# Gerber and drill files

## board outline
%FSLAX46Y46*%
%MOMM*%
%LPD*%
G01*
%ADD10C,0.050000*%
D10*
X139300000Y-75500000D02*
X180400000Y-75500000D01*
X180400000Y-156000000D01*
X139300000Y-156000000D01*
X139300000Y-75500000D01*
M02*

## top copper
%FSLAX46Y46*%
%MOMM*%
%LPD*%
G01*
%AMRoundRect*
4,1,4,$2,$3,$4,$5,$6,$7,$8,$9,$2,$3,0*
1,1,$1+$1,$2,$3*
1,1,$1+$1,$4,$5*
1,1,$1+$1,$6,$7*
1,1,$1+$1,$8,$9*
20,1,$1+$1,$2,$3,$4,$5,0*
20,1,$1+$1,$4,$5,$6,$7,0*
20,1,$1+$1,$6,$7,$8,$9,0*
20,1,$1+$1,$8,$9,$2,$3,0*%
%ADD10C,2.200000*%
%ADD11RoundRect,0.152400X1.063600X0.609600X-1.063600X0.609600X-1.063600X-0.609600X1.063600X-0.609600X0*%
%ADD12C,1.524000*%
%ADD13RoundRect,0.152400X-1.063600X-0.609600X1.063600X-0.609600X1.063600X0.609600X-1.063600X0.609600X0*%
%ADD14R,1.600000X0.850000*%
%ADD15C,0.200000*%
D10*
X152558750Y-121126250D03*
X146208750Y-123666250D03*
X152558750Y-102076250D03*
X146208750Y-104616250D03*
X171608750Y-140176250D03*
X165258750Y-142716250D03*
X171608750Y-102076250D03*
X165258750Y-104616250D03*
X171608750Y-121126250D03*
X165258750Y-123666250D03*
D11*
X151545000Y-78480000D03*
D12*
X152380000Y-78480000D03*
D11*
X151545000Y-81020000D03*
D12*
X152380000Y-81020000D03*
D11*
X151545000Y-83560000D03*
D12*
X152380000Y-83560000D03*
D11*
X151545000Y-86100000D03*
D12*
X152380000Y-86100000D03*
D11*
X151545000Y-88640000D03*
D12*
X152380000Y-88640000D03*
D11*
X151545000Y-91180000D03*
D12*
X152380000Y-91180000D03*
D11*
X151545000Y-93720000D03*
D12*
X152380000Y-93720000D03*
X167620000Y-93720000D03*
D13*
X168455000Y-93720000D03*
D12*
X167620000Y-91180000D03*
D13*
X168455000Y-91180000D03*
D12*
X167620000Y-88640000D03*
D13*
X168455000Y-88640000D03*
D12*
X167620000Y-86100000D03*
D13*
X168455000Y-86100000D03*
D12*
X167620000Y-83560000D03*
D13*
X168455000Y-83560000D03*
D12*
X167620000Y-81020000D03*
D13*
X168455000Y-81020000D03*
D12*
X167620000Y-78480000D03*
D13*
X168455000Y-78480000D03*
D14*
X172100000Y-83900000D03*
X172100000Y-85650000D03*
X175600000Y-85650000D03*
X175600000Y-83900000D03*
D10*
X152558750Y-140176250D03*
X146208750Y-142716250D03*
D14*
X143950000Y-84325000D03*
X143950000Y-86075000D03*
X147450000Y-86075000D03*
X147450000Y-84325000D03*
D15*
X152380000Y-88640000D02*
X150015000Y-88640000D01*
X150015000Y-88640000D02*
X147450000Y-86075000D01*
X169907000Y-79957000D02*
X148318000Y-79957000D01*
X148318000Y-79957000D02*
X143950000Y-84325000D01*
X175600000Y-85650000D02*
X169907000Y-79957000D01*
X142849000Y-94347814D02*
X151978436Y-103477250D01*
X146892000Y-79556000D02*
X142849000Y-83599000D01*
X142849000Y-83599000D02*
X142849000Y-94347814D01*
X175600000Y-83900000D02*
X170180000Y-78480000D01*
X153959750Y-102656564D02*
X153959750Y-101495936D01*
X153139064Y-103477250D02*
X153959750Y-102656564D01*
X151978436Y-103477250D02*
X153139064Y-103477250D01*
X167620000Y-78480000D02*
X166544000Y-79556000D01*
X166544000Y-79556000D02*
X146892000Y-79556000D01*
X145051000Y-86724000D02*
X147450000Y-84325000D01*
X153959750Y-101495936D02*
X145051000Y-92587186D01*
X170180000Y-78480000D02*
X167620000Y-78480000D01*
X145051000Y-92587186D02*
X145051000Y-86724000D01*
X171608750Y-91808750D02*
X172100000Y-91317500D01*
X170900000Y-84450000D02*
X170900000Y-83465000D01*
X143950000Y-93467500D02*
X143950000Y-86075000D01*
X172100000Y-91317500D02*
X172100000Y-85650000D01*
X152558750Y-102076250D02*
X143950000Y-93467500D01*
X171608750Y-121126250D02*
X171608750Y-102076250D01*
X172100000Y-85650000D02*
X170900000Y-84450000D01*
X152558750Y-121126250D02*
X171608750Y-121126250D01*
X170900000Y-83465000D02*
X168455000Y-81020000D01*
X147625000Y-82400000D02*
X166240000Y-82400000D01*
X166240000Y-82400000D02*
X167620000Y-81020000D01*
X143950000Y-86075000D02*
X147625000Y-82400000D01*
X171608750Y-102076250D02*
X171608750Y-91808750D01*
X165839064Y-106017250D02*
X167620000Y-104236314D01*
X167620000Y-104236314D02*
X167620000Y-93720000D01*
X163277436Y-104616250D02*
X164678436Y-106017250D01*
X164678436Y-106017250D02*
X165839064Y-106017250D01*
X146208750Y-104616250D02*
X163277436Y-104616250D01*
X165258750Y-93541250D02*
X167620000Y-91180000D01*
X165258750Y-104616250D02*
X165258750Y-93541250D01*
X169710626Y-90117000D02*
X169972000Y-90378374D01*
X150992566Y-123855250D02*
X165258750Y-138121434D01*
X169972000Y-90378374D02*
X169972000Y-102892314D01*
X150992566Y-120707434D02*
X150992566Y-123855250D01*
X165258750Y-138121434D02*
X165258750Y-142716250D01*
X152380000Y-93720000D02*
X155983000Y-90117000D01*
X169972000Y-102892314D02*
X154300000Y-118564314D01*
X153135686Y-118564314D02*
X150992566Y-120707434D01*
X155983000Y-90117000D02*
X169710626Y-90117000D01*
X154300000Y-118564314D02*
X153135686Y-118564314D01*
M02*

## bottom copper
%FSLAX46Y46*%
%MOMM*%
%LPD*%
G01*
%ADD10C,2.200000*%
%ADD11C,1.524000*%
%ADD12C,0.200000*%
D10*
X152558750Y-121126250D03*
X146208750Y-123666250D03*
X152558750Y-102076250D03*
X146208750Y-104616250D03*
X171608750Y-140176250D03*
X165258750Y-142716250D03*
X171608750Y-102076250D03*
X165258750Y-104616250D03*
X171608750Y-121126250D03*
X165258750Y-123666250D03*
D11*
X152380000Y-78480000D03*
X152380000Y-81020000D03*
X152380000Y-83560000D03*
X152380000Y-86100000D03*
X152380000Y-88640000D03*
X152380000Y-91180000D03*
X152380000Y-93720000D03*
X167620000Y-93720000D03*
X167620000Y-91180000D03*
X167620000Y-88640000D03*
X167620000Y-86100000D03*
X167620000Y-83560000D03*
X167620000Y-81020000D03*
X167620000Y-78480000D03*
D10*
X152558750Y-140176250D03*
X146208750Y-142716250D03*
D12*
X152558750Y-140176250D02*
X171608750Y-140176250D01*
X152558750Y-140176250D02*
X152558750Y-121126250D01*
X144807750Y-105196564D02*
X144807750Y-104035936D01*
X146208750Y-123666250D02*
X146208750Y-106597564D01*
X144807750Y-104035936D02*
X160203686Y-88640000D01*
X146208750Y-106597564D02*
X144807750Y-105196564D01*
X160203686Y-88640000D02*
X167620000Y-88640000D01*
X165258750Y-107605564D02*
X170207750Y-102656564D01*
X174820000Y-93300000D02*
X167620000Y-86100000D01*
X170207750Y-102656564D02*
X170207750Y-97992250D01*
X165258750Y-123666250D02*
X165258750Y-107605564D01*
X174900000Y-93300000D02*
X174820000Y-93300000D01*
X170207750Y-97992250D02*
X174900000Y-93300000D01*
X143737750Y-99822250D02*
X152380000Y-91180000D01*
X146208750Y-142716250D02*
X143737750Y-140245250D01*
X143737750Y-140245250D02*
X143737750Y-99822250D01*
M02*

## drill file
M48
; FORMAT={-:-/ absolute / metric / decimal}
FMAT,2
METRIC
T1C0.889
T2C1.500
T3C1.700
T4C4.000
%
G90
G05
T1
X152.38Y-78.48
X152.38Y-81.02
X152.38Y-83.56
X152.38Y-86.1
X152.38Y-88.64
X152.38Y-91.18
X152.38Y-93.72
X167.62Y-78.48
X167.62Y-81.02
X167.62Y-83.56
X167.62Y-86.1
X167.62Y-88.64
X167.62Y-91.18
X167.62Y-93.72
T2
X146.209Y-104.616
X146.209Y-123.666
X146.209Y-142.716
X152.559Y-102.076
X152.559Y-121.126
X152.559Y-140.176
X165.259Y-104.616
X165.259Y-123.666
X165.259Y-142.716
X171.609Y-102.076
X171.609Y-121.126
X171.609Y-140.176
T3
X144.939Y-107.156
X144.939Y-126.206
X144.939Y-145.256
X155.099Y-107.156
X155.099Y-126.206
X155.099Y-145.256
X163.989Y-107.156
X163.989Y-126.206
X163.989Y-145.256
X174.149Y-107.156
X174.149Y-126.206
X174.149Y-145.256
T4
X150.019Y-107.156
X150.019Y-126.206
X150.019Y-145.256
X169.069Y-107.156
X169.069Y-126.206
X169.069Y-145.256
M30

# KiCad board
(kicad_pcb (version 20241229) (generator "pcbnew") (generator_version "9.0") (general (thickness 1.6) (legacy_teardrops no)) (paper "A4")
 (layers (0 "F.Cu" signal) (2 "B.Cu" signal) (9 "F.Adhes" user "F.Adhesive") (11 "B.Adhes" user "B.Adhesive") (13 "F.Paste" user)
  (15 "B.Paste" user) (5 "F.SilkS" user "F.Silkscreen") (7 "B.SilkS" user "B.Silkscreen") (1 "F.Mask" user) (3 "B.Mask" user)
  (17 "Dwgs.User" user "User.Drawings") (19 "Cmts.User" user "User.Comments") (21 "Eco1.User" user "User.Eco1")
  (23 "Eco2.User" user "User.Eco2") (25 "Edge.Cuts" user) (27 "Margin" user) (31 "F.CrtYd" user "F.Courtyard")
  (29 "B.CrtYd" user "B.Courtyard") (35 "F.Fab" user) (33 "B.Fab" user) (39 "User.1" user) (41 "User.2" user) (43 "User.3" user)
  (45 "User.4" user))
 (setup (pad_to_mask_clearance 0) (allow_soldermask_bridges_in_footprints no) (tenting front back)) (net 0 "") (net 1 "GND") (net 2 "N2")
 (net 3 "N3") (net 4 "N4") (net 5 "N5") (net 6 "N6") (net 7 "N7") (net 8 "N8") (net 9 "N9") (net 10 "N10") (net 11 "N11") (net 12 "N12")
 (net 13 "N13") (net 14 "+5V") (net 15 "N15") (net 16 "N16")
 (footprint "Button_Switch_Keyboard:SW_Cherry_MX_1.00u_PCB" (layer "F.Cu") (at 152.55875 121.12625)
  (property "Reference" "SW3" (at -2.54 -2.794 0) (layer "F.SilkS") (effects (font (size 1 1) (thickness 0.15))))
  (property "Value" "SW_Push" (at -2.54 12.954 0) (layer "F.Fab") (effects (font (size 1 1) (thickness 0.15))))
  (pad "" np_thru_hole circle (at -7.62 5.08) (size 1.7 1.7) (drill 1.7) (layers "*.Cu" "*.Mask"))
  (pad "" np_thru_hole circle (at -2.54 5.08) (size 4 4) (drill 4) (layers "*.Cu" "*.Mask"))
  (pad "" np_thru_hole circle (at 2.54 5.08) (size 1.7 1.7) (drill 1.7) (layers "*.Cu" "*.Mask"))
  (pad "1" thru_hole circle (at 0 0) (size 2.2 2.2) (drill 1.5) (layers "*.Cu" "*.Mask") (remove_unused_layers no) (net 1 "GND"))
  (pad "2" thru_hole circle (at -6.35 2.54) (size 2.2 2.2) (drill 1.5) (layers "*.Cu" "*.Mask") (remove_unused_layers no) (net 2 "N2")))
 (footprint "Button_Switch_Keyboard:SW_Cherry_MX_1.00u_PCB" (layer "F.Cu") (at 152.55875 102.07625)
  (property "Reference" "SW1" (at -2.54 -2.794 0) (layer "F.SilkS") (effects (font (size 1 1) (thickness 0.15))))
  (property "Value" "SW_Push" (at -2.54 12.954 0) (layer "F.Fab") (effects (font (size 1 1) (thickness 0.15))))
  (pad "" np_thru_hole circle (at -7.62 5.08) (size 1.7 1.7) (drill 1.7) (layers "*.Cu" "*.Mask"))
  (pad "" np_thru_hole circle (at -2.54 5.08) (size 4 4) (drill 4) (layers "*.Cu" "*.Mask"))
  (pad "" np_thru_hole circle (at 2.54 5.08) (size 1.7 1.7) (drill 1.7) (layers "*.Cu" "*.Mask"))
  (pad "1" thru_hole circle (at 0 0) (size 2.2 2.2) (drill 1.5) (layers "*.Cu" "*.Mask") (remove_unused_layers no) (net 1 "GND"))
  (pad "2" thru_hole circle (at -6.35 2.54) (size 2.2 2.2) (drill 1.5) (layers "*.Cu" "*.Mask") (remove_unused_layers no) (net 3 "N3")))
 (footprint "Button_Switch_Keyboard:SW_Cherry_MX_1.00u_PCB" (layer "F.Cu") (at 171.60875 140.17625)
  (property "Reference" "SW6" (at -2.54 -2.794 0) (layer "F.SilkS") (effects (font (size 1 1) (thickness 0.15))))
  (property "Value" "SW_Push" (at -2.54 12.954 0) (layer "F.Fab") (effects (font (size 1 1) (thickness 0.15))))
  (pad "" np_thru_hole circle (at -7.62 5.08) (size 1.7 1.7) (drill 1.7) (layers "*.Cu" "*.Mask"))
  (pad "" np_thru_hole circle (at -2.54 5.08) (size 4 4) (drill 4) (layers "*.Cu" "*.Mask"))
  (pad "" np_thru_hole circle (at 2.54 5.08) (size 1.7 1.7) (drill 1.7) (layers "*.Cu" "*.Mask"))
  (pad "1" thru_hole circle (at 0 0) (size 2.2 2.2) (drill 1.5) (layers "*.Cu" "*.Mask") (remove_unused_layers no) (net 1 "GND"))
  (pad "2" thru_hole circle (at -6.35 2.54) (size 2.2 2.2) (drill 1.5) (layers "*.Cu" "*.Mask") (remove_unused_layers no) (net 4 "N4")))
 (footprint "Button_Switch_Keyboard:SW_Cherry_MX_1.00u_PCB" (layer "F.Cu") (at 171.60875 102.07625)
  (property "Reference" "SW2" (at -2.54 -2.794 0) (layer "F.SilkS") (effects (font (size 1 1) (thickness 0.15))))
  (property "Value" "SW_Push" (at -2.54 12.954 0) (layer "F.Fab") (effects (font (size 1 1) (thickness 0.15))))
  (pad "" np_thru_hole circle (at -7.62 5.08) (size 1.7 1.7) (drill 1.7) (layers "*.Cu" "*.Mask"))
  (pad "" np_thru_hole circle (at -2.54 5.08) (size 4 4) (drill 4) (layers "*.Cu" "*.Mask"))
  (pad "" np_thru_hole circle (at 2.54 5.08) (size 1.7 1.7) (drill 1.7) (layers "*.Cu" "*.Mask"))
  (pad "1" thru_hole circle (at 0 0) (size 2.2 2.2) (drill 1.5) (layers "*.Cu" "*.Mask") (remove_unused_layers no) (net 1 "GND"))
  (pad "2" thru_hole circle (at -6.35 2.54) (size 2.2 2.2) (drill 1.5) (layers "*.Cu" "*.Mask") (remove_unused_layers no) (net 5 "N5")))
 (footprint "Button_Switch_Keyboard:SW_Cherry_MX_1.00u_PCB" (layer "F.Cu") (at 171.60875 121.12625)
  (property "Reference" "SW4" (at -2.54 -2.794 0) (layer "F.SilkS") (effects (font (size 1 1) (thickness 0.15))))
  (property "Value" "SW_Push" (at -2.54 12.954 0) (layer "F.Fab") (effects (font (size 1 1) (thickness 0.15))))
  (pad "" np_thru_hole circle (at -7.62 5.08) (size 1.7 1.7) (drill 1.7) (layers "*.Cu" "*.Mask"))
  (pad "" np_thru_hole circle (at -2.54 5.08) (size 4 4) (drill 4) (layers "*.Cu" "*.Mask"))
  (pad "" np_thru_hole circle (at 2.54 5.08) (size 1.7 1.7) (drill 1.7) (layers "*.Cu" "*.Mask"))
  (pad "1" thru_hole circle (at 0 0) (size 2.2 2.2) (drill 1.5) (layers "*.Cu" "*.Mask") (remove_unused_layers no) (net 1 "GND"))
  (pad "2" thru_hole circle (at -6.35 2.54) (size 2.2 2.2) (drill 1.5) (layers "*.Cu" "*.Mask") (remove_unused_layers no) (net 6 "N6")))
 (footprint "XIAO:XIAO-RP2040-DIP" (layer "F.Cu") (at 160 86.1)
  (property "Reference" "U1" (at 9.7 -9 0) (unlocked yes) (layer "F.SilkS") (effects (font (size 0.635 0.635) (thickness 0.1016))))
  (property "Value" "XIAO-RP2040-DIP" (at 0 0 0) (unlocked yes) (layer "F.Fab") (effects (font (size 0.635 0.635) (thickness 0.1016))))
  (pad "1" smd roundrect (at -8.455 -7.62 180) (size 2.432 1.524) (layers "F.Cu" "F.Mask") (roundrect_rratio 0.1) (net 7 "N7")
   (thermal_bridge_angle 45))
  (pad "1" thru_hole circle (at -7.62 -7.62 180) (size 1.524 1.524) (drill 0.889) (layers "*.Cu" "*.Mask") (remove_unused_layers no)
   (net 7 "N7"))
  (pad "2" smd roundrect (at -8.455 -5.08 180) (size 2.432 1.524) (layers "F.Cu" "F.Mask") (roundrect_rratio 0.1) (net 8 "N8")
   (thermal_bridge_angle 45))
  (pad "2" thru_hole circle (at -7.62 -5.08 180) (size 1.524 1.524) (drill 0.889) (layers "*.Cu" "*.Mask") (remove_unused_layers no)
   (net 8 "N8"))
  (pad "3" smd roundrect (at -8.455 -2.54 180) (size 2.432 1.524) (layers "F.Cu" "F.Mask") (roundrect_rratio 0.1) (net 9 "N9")
   (thermal_bridge_angle 45))
  (pad "3" thru_hole circle (at -7.62 -2.54 180) (size 1.524 1.524) (drill 0.889) (layers "*.Cu" "*.Mask") (remove_unused_layers no)
   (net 9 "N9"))
  (pad "4" smd roundrect (at -8.455 0 180) (size 2.432 1.524) (layers "F.Cu" "F.Mask") (roundrect_rratio 0.1) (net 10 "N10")
   (thermal_bridge_angle 45))
  (pad "4" thru_hole circle (at -7.62 0 180) (size 1.524 1.524) (drill 0.889) (layers "*.Cu" "*.Mask") (remove_unused_layers no)
   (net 10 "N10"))
  (pad "5" smd roundrect (at -8.455 2.54 180) (size 2.432 1.524) (layers "F.Cu" "F.Mask") (roundrect_rratio 0.1) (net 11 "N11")
   (thermal_bridge_angle 45))
  (pad "5" thru_hole circle (at -7.62 2.54 180) (size 1.524 1.524) (drill 0.889) (layers "*.Cu" "*.Mask") (remove_unused_layers no)
   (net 11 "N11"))
  (pad "6" smd roundrect (at -8.455 5.08 180) (size 2.432 1.524) (layers "F.Cu" "F.Mask") (roundrect_rratio 0.1) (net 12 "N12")
   (thermal_bridge_angle 45))
  (pad "6" thru_hole circle (at -7.62 5.08 180) (size 1.524 1.524) (drill 0.889) (layers "*.Cu" "*.Mask") (remove_unused_layers no)
   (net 12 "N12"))
  (pad "7" smd roundrect (at -8.455 7.62 180) (size 2.432 1.524) (layers "F.Cu" "F.Mask") (roundrect_rratio 0.1) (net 4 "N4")
   (thermal_bridge_angle 45))
  (pad "7" thru_hole circle (at -7.62 7.62 180) (size 1.524 1.524) (drill 0.889) (layers "*.Cu" "*.Mask") (remove_unused_layers no)
   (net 4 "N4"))
  (pad "8" thru_hole circle (at 7.62 7.62) (size 1.524 1.524) (drill 0.889) (layers "*.Cu" "*.Mask") (remove_unused_layers no) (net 3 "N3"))
  (pad "8" smd roundrect (at 8.455 7.62) (size 2.432 1.524) (layers "F.Cu" "F.Mask") (roundrect_rratio 0.1) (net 3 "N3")
   (thermal_bridge_angle 45))
  (pad "9" thru_hole circle (at 7.62 5.08) (size 1.524 1.524) (drill 0.889) (layers "*.Cu" "*.Mask") (remove_unused_layers no) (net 5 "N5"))
  (pad "9" smd roundrect (at 8.455 5.08) (size 2.432 1.524) (layers "F.Cu" "F.Mask") (roundrect_rratio 0.1) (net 5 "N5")
   (thermal_bridge_angle 45))
  (pad "10" thru_hole circle (at 7.62 2.54) (size 1.524 1.524) (drill 0.889) (layers "*.Cu" "*.Mask") (remove_unused_layers no) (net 2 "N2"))
  (pad "10" smd roundrect (at 8.455 2.54) (size 2.432 1.524) (layers "F.Cu" "F.Mask") (roundrect_rratio 0.1) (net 2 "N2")
   (thermal_bridge_angle 45))
  (pad "11" thru_hole circle (at 7.62 0) (size 1.524 1.524) (drill 0.889) (layers "*.Cu" "*.Mask") (remove_unused_layers no) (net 6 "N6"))
  (pad "11" smd roundrect (at 8.455 0) (size 2.432 1.524) (layers "F.Cu" "F.Mask") (roundrect_rratio 0.1) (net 6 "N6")
   (thermal_bridge_angle 45))
  (pad "12" thru_hole circle (at 7.62 -2.54) (size 1.524 1.524) (drill 0.889) (layers "*.Cu" "*.Mask") (remove_unused_layers no)
   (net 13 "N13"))
  (pad "12" smd roundrect (at 8.455 -2.54) (size 2.432 1.524) (layers "F.Cu" "F.Mask") (roundrect_rratio 0.1) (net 13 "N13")
   (thermal_bridge_angle 45))
  (pad "13" thru_hole circle (at 7.62 -5.08) (size 1.524 1.524) (drill 0.889) (layers "*.Cu" "*.Mask") (remove_unused_layers no)
   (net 1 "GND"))
  (pad "13" smd roundrect (at 8.455 -5.08) (size 2.432 1.524) (layers "F.Cu" "F.Mask") (roundrect_rratio 0.1) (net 1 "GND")
   (thermal_bridge_angle 45))
  (pad "14" thru_hole circle (at 7.62 -7.62) (size 1.524 1.524) (drill 0.889) (layers "*.Cu" "*.Mask") (remove_unused_layers no)
   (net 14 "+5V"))
  (pad "14" smd roundrect (at 8.455 -7.62) (size 2.432 1.524) (layers "F.Cu" "F.Mask") (roundrect_rratio 0.1) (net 14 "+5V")
   (thermal_bridge_angle 45)))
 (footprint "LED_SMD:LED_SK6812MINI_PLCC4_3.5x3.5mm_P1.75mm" (layer "F.Cu") (at 173.85 84.775)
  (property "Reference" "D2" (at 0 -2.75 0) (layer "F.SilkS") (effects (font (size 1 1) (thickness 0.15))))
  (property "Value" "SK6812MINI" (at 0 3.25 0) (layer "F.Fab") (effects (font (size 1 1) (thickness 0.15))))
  (pad "1" smd rect (at -1.75 -0.875) (size 1.6 0.85) (layers "F.Cu" "F.Mask" "F.Paste") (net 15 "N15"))
  (pad "2" smd rect (at -1.75 0.875) (size 1.6 0.85) (layers "F.Cu" "F.Mask" "F.Paste") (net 1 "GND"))
  (pad "3" smd rect (at 1.75 0.875) (size 1.6 0.85) (layers "F.Cu" "F.Mask" "F.Paste") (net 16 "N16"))
  (pad "4" smd rect (at 1.75 -0.875) (size 1.6 0.85) (layers "F.Cu" "F.Mask" "F.Paste") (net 14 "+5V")))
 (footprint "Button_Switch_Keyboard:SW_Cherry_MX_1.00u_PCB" (layer "F.Cu") (at 152.55875 140.17625)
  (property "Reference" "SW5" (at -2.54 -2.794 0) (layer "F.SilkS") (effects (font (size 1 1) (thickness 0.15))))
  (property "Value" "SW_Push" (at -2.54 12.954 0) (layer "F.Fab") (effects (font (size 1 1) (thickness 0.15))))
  (pad "" np_thru_hole circle (at -7.62 5.08) (size 1.7 1.7) (drill 1.7) (layers "*.Cu" "*.Mask"))
  (pad "" np_thru_hole circle (at -2.54 5.08) (size 4 4) (drill 4) (layers "*.Cu" "*.Mask"))
  (pad "" np_thru_hole circle (at 2.54 5.08) (size 1.7 1.7) (drill 1.7) (layers "*.Cu" "*.Mask"))
  (pad "1" thru_hole circle (at 0 0) (size 2.2 2.2) (drill 1.5) (layers "*.Cu" "*.Mask") (remove_unused_layers no) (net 1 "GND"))
  (pad "2" thru_hole circle (at -6.35 2.54) (size 2.2 2.2) (drill 1.5) (layers "*.Cu" "*.Mask") (remove_unused_layers no) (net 12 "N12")))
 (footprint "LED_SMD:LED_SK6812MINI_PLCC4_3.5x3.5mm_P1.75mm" (layer "F.Cu") (at 145.7 85.2)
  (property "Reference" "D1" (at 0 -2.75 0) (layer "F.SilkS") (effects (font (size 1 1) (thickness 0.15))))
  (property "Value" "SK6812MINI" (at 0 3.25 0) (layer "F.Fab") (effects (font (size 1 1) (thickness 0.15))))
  (pad "1" smd rect (at -1.75 -0.875) (size 1.6 0.85) (layers "F.Cu" "F.Mask" "F.Paste") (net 16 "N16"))
  (pad "2" smd rect (at -1.75 0.875) (size 1.6 0.85) (layers "F.Cu" "F.Mask" "F.Paste") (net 1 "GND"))
  (pad "3" smd rect (at 1.75 0.875) (size 1.6 0.85) (layers "F.Cu" "F.Mask" "F.Paste") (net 11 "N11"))
  (pad "4" smd rect (at 1.75 -0.875) (size 1.6 0.85) (layers "F.Cu" "F.Mask" "F.Paste") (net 14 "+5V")))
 (gr_rect (start 139.3 75.5) (end 180.4 156) (stroke (width 0.05) (type default)) (fill no) (layer "Edge.Cuts"))
 (segment (start 152.38 88.64) (end 150.015 88.64) (width 0.2) (layer "F.Cu") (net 11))
 (segment (start 150.015 88.64) (end 147.45 86.075) (width 0.2) (layer "F.Cu") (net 11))
 (segment (start 169.907 79.957) (end 148.318 79.957) (width 0.2) (layer "F.Cu") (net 16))
 (segment (start 148.318 79.957) (end 143.95 84.325) (width 0.2) (layer "F.Cu") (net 16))
 (segment (start 175.6 85.65) (end 169.907 79.957) (width 0.2) (layer "F.Cu") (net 16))
 (segment (start 142.849 94.347814) (end 151.978436 103.47725) (width 0.2) (layer "F.Cu") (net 14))
 (segment (start 146.892 79.556) (end 142.849 83.599) (width 0.2) (layer "F.Cu") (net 14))
 (segment (start 142.849 83.599) (end 142.849 94.347814) (width 0.2) (layer "F.Cu") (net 14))
 (segment (start 175.6 83.9) (end 170.18 78.48) (width 0.2) (layer "F.Cu") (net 14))
 (segment (start 153.95975 102.656564) (end 153.95975 101.495936) (width 0.2) (layer "F.Cu") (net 14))
 (segment (start 153.139064 103.47725) (end 153.95975 102.656564) (width 0.2) (layer "F.Cu") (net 14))
 (segment (start 151.978436 103.47725) (end 153.139064 103.47725) (width 0.2) (layer "F.Cu") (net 14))
 (segment (start 167.62 78.48) (end 166.544 79.556) (width 0.2) (layer "F.Cu") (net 14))
 (segment (start 166.544 79.556) (end 146.892 79.556) (width 0.2) (layer "F.Cu") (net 14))
 (segment (start 145.051 86.724) (end 147.45 84.325) (width 0.2) (layer "F.Cu") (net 14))
 (segment (start 153.95975 101.495936) (end 145.051 92.587186) (width 0.2) (layer "F.Cu") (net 14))
 (segment (start 170.18 78.48) (end 167.62 78.48) (width 0.2) (layer "F.Cu") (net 14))
 (segment (start 145.051 92.587186) (end 145.051 86.724) (width 0.2) (layer "F.Cu") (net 14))
 (segment (start 171.60875 91.80875) (end 172.1 91.3175) (width 0.2) (layer "F.Cu") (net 1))
 (segment (start 170.9 84.45) (end 170.9 83.465) (width 0.2) (layer "F.Cu") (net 1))
 (segment (start 143.95 93.4675) (end 143.95 86.075) (width 0.2) (layer "F.Cu") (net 1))
 (segment (start 172.1 91.3175) (end 172.1 85.65) (width 0.2) (layer "F.Cu") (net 1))
 (segment (start 152.55875 102.07625) (end 143.95 93.4675) (width 0.2) (layer "F.Cu") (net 1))
 (segment (start 171.60875 121.12625) (end 171.60875 102.07625) (width 0.2) (layer "F.Cu") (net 1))
 (segment (start 172.1 85.65) (end 170.9 84.45) (width 0.2) (layer "F.Cu") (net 1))
 (segment (start 152.55875 121.12625) (end 171.60875 121.12625) (width 0.2) (layer "F.Cu") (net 1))
 (segment (start 170.9 83.465) (end 168.455 81.02) (width 0.2) (layer "F.Cu") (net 1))
 (segment (start 147.625 82.4) (end 166.24 82.4) (width 0.2) (layer "F.Cu") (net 1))
 (segment (start 166.24 82.4) (end 167.62 81.02) (width 0.2) (layer "F.Cu") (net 1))
 (segment (start 143.95 86.075) (end 147.625 82.4) (width 0.2) (layer "F.Cu") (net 1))
 (segment (start 171.60875 102.07625) (end 171.60875 91.80875) (width 0.2) (layer "F.Cu") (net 1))
 (segment (start 152.55875 140.17625) (end 171.60875 140.17625) (width 0.2) (layer "B.Cu") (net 1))
 (segment (start 152.55875 140.17625) (end 152.55875 121.12625) (width 0.2) (layer "B.Cu") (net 1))
 (segment (start 165.839064 106.01725) (end 167.62 104.236314) (width 0.2) (layer "F.Cu") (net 3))
 (segment (start 167.62 104.236314) (end 167.62 93.72) (width 0.2) (layer "F.Cu") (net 3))
 (segment (start 163.277436 104.61625) (end 164.678436 106.01725) (width 0.2) (layer "F.Cu") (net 3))
 (segment (start 164.678436 106.01725) (end 165.839064 106.01725) (width 0.2) (layer "F.Cu") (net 3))
 (segment (start 146.20875 104.61625) (end 163.277436 104.61625) (width 0.2) (layer "F.Cu") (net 3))
 (segment (start 165.25875 93.54125) (end 167.62 91.18) (width 0.2) (layer "F.Cu") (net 5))
 (segment (start 165.25875 104.61625) (end 165.25875 93.54125) (width 0.2) (layer "F.Cu") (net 5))
 (segment (start 144.80775 105.196564) (end 144.80775 104.035936) (width 0.2) (layer "B.Cu") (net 2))
 (segment (start 146.20875 123.66625) (end 146.20875 106.597564) (width 0.2) (layer "B.Cu") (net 2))
 (segment (start 144.80775 104.035936) (end 160.203686 88.64) (width 0.2) (layer "B.Cu") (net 2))
 (segment (start 146.20875 106.597564) (end 144.80775 105.196564) (width 0.2) (layer "B.Cu") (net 2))
 (segment (start 160.203686 88.64) (end 167.62 88.64) (width 0.2) (layer "B.Cu") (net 2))
 (segment (start 165.25875 107.605564) (end 170.20775 102.656564) (width 0.2) (layer "B.Cu") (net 6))
 (segment (start 174.82 93.3) (end 167.62 86.1) (width 0.2) (layer "B.Cu") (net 6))
 (segment (start 170.20775 102.656564) (end 170.20775 97.99225) (width 0.2) (layer "B.Cu") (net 6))
 (segment (start 165.25875 123.66625) (end 165.25875 107.605564) (width 0.2) (layer "B.Cu") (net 6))
 (segment (start 174.9 93.3) (end 174.82 93.3) (width 0.2) (layer "B.Cu") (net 6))
 (segment (start 170.20775 97.99225) (end 174.9 93.3) (width 0.2) (layer "B.Cu") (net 6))
 (segment (start 143.73775 99.82225) (end 152.38 91.18) (width 0.2) (layer "B.Cu") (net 12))
 (segment (start 146.20875 142.71625) (end 143.73775 140.24525) (width 0.2) (layer "B.Cu") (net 12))
 (segment (start 143.73775 140.24525) (end 143.73775 99.82225) (width 0.2) (layer "B.Cu") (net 12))
 (segment (start 169.710626 90.117) (end 169.972 90.378374) (width 0.2) (layer "F.Cu") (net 4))
 (segment (start 150.992566 123.85525) (end 165.25875 138.121434) (width 0.2) (layer "F.Cu") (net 4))
 (segment (start 169.972 90.378374) (end 169.972 102.892314) (width 0.2) (layer "F.Cu") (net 4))
 (segment (start 150.992566 120.707434) (end 150.992566 123.85525) (width 0.2) (layer "F.Cu") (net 4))
 (segment (start 165.25875 138.121434) (end 165.25875 142.71625) (width 0.2) (layer "F.Cu") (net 4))
 (segment (start 152.38 93.72) (end 155.983 90.117) (width 0.2) (layer "F.Cu") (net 4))
 (segment (start 169.972 102.892314) (end 154.3 118.564314) (width 0.2) (layer "F.Cu") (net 4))
 (segment (start 153.135686 118.564314) (end 150.992566 120.707434) (width 0.2) (layer "F.Cu") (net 4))
 (segment (start 155.983 90.117) (end 169.710626 90.117) (width 0.2) (layer "F.Cu") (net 4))
 (segment (start 154.3 118.564314) (end 153.135686 118.564314) (width 0.2) (layer "F.Cu") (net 4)))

